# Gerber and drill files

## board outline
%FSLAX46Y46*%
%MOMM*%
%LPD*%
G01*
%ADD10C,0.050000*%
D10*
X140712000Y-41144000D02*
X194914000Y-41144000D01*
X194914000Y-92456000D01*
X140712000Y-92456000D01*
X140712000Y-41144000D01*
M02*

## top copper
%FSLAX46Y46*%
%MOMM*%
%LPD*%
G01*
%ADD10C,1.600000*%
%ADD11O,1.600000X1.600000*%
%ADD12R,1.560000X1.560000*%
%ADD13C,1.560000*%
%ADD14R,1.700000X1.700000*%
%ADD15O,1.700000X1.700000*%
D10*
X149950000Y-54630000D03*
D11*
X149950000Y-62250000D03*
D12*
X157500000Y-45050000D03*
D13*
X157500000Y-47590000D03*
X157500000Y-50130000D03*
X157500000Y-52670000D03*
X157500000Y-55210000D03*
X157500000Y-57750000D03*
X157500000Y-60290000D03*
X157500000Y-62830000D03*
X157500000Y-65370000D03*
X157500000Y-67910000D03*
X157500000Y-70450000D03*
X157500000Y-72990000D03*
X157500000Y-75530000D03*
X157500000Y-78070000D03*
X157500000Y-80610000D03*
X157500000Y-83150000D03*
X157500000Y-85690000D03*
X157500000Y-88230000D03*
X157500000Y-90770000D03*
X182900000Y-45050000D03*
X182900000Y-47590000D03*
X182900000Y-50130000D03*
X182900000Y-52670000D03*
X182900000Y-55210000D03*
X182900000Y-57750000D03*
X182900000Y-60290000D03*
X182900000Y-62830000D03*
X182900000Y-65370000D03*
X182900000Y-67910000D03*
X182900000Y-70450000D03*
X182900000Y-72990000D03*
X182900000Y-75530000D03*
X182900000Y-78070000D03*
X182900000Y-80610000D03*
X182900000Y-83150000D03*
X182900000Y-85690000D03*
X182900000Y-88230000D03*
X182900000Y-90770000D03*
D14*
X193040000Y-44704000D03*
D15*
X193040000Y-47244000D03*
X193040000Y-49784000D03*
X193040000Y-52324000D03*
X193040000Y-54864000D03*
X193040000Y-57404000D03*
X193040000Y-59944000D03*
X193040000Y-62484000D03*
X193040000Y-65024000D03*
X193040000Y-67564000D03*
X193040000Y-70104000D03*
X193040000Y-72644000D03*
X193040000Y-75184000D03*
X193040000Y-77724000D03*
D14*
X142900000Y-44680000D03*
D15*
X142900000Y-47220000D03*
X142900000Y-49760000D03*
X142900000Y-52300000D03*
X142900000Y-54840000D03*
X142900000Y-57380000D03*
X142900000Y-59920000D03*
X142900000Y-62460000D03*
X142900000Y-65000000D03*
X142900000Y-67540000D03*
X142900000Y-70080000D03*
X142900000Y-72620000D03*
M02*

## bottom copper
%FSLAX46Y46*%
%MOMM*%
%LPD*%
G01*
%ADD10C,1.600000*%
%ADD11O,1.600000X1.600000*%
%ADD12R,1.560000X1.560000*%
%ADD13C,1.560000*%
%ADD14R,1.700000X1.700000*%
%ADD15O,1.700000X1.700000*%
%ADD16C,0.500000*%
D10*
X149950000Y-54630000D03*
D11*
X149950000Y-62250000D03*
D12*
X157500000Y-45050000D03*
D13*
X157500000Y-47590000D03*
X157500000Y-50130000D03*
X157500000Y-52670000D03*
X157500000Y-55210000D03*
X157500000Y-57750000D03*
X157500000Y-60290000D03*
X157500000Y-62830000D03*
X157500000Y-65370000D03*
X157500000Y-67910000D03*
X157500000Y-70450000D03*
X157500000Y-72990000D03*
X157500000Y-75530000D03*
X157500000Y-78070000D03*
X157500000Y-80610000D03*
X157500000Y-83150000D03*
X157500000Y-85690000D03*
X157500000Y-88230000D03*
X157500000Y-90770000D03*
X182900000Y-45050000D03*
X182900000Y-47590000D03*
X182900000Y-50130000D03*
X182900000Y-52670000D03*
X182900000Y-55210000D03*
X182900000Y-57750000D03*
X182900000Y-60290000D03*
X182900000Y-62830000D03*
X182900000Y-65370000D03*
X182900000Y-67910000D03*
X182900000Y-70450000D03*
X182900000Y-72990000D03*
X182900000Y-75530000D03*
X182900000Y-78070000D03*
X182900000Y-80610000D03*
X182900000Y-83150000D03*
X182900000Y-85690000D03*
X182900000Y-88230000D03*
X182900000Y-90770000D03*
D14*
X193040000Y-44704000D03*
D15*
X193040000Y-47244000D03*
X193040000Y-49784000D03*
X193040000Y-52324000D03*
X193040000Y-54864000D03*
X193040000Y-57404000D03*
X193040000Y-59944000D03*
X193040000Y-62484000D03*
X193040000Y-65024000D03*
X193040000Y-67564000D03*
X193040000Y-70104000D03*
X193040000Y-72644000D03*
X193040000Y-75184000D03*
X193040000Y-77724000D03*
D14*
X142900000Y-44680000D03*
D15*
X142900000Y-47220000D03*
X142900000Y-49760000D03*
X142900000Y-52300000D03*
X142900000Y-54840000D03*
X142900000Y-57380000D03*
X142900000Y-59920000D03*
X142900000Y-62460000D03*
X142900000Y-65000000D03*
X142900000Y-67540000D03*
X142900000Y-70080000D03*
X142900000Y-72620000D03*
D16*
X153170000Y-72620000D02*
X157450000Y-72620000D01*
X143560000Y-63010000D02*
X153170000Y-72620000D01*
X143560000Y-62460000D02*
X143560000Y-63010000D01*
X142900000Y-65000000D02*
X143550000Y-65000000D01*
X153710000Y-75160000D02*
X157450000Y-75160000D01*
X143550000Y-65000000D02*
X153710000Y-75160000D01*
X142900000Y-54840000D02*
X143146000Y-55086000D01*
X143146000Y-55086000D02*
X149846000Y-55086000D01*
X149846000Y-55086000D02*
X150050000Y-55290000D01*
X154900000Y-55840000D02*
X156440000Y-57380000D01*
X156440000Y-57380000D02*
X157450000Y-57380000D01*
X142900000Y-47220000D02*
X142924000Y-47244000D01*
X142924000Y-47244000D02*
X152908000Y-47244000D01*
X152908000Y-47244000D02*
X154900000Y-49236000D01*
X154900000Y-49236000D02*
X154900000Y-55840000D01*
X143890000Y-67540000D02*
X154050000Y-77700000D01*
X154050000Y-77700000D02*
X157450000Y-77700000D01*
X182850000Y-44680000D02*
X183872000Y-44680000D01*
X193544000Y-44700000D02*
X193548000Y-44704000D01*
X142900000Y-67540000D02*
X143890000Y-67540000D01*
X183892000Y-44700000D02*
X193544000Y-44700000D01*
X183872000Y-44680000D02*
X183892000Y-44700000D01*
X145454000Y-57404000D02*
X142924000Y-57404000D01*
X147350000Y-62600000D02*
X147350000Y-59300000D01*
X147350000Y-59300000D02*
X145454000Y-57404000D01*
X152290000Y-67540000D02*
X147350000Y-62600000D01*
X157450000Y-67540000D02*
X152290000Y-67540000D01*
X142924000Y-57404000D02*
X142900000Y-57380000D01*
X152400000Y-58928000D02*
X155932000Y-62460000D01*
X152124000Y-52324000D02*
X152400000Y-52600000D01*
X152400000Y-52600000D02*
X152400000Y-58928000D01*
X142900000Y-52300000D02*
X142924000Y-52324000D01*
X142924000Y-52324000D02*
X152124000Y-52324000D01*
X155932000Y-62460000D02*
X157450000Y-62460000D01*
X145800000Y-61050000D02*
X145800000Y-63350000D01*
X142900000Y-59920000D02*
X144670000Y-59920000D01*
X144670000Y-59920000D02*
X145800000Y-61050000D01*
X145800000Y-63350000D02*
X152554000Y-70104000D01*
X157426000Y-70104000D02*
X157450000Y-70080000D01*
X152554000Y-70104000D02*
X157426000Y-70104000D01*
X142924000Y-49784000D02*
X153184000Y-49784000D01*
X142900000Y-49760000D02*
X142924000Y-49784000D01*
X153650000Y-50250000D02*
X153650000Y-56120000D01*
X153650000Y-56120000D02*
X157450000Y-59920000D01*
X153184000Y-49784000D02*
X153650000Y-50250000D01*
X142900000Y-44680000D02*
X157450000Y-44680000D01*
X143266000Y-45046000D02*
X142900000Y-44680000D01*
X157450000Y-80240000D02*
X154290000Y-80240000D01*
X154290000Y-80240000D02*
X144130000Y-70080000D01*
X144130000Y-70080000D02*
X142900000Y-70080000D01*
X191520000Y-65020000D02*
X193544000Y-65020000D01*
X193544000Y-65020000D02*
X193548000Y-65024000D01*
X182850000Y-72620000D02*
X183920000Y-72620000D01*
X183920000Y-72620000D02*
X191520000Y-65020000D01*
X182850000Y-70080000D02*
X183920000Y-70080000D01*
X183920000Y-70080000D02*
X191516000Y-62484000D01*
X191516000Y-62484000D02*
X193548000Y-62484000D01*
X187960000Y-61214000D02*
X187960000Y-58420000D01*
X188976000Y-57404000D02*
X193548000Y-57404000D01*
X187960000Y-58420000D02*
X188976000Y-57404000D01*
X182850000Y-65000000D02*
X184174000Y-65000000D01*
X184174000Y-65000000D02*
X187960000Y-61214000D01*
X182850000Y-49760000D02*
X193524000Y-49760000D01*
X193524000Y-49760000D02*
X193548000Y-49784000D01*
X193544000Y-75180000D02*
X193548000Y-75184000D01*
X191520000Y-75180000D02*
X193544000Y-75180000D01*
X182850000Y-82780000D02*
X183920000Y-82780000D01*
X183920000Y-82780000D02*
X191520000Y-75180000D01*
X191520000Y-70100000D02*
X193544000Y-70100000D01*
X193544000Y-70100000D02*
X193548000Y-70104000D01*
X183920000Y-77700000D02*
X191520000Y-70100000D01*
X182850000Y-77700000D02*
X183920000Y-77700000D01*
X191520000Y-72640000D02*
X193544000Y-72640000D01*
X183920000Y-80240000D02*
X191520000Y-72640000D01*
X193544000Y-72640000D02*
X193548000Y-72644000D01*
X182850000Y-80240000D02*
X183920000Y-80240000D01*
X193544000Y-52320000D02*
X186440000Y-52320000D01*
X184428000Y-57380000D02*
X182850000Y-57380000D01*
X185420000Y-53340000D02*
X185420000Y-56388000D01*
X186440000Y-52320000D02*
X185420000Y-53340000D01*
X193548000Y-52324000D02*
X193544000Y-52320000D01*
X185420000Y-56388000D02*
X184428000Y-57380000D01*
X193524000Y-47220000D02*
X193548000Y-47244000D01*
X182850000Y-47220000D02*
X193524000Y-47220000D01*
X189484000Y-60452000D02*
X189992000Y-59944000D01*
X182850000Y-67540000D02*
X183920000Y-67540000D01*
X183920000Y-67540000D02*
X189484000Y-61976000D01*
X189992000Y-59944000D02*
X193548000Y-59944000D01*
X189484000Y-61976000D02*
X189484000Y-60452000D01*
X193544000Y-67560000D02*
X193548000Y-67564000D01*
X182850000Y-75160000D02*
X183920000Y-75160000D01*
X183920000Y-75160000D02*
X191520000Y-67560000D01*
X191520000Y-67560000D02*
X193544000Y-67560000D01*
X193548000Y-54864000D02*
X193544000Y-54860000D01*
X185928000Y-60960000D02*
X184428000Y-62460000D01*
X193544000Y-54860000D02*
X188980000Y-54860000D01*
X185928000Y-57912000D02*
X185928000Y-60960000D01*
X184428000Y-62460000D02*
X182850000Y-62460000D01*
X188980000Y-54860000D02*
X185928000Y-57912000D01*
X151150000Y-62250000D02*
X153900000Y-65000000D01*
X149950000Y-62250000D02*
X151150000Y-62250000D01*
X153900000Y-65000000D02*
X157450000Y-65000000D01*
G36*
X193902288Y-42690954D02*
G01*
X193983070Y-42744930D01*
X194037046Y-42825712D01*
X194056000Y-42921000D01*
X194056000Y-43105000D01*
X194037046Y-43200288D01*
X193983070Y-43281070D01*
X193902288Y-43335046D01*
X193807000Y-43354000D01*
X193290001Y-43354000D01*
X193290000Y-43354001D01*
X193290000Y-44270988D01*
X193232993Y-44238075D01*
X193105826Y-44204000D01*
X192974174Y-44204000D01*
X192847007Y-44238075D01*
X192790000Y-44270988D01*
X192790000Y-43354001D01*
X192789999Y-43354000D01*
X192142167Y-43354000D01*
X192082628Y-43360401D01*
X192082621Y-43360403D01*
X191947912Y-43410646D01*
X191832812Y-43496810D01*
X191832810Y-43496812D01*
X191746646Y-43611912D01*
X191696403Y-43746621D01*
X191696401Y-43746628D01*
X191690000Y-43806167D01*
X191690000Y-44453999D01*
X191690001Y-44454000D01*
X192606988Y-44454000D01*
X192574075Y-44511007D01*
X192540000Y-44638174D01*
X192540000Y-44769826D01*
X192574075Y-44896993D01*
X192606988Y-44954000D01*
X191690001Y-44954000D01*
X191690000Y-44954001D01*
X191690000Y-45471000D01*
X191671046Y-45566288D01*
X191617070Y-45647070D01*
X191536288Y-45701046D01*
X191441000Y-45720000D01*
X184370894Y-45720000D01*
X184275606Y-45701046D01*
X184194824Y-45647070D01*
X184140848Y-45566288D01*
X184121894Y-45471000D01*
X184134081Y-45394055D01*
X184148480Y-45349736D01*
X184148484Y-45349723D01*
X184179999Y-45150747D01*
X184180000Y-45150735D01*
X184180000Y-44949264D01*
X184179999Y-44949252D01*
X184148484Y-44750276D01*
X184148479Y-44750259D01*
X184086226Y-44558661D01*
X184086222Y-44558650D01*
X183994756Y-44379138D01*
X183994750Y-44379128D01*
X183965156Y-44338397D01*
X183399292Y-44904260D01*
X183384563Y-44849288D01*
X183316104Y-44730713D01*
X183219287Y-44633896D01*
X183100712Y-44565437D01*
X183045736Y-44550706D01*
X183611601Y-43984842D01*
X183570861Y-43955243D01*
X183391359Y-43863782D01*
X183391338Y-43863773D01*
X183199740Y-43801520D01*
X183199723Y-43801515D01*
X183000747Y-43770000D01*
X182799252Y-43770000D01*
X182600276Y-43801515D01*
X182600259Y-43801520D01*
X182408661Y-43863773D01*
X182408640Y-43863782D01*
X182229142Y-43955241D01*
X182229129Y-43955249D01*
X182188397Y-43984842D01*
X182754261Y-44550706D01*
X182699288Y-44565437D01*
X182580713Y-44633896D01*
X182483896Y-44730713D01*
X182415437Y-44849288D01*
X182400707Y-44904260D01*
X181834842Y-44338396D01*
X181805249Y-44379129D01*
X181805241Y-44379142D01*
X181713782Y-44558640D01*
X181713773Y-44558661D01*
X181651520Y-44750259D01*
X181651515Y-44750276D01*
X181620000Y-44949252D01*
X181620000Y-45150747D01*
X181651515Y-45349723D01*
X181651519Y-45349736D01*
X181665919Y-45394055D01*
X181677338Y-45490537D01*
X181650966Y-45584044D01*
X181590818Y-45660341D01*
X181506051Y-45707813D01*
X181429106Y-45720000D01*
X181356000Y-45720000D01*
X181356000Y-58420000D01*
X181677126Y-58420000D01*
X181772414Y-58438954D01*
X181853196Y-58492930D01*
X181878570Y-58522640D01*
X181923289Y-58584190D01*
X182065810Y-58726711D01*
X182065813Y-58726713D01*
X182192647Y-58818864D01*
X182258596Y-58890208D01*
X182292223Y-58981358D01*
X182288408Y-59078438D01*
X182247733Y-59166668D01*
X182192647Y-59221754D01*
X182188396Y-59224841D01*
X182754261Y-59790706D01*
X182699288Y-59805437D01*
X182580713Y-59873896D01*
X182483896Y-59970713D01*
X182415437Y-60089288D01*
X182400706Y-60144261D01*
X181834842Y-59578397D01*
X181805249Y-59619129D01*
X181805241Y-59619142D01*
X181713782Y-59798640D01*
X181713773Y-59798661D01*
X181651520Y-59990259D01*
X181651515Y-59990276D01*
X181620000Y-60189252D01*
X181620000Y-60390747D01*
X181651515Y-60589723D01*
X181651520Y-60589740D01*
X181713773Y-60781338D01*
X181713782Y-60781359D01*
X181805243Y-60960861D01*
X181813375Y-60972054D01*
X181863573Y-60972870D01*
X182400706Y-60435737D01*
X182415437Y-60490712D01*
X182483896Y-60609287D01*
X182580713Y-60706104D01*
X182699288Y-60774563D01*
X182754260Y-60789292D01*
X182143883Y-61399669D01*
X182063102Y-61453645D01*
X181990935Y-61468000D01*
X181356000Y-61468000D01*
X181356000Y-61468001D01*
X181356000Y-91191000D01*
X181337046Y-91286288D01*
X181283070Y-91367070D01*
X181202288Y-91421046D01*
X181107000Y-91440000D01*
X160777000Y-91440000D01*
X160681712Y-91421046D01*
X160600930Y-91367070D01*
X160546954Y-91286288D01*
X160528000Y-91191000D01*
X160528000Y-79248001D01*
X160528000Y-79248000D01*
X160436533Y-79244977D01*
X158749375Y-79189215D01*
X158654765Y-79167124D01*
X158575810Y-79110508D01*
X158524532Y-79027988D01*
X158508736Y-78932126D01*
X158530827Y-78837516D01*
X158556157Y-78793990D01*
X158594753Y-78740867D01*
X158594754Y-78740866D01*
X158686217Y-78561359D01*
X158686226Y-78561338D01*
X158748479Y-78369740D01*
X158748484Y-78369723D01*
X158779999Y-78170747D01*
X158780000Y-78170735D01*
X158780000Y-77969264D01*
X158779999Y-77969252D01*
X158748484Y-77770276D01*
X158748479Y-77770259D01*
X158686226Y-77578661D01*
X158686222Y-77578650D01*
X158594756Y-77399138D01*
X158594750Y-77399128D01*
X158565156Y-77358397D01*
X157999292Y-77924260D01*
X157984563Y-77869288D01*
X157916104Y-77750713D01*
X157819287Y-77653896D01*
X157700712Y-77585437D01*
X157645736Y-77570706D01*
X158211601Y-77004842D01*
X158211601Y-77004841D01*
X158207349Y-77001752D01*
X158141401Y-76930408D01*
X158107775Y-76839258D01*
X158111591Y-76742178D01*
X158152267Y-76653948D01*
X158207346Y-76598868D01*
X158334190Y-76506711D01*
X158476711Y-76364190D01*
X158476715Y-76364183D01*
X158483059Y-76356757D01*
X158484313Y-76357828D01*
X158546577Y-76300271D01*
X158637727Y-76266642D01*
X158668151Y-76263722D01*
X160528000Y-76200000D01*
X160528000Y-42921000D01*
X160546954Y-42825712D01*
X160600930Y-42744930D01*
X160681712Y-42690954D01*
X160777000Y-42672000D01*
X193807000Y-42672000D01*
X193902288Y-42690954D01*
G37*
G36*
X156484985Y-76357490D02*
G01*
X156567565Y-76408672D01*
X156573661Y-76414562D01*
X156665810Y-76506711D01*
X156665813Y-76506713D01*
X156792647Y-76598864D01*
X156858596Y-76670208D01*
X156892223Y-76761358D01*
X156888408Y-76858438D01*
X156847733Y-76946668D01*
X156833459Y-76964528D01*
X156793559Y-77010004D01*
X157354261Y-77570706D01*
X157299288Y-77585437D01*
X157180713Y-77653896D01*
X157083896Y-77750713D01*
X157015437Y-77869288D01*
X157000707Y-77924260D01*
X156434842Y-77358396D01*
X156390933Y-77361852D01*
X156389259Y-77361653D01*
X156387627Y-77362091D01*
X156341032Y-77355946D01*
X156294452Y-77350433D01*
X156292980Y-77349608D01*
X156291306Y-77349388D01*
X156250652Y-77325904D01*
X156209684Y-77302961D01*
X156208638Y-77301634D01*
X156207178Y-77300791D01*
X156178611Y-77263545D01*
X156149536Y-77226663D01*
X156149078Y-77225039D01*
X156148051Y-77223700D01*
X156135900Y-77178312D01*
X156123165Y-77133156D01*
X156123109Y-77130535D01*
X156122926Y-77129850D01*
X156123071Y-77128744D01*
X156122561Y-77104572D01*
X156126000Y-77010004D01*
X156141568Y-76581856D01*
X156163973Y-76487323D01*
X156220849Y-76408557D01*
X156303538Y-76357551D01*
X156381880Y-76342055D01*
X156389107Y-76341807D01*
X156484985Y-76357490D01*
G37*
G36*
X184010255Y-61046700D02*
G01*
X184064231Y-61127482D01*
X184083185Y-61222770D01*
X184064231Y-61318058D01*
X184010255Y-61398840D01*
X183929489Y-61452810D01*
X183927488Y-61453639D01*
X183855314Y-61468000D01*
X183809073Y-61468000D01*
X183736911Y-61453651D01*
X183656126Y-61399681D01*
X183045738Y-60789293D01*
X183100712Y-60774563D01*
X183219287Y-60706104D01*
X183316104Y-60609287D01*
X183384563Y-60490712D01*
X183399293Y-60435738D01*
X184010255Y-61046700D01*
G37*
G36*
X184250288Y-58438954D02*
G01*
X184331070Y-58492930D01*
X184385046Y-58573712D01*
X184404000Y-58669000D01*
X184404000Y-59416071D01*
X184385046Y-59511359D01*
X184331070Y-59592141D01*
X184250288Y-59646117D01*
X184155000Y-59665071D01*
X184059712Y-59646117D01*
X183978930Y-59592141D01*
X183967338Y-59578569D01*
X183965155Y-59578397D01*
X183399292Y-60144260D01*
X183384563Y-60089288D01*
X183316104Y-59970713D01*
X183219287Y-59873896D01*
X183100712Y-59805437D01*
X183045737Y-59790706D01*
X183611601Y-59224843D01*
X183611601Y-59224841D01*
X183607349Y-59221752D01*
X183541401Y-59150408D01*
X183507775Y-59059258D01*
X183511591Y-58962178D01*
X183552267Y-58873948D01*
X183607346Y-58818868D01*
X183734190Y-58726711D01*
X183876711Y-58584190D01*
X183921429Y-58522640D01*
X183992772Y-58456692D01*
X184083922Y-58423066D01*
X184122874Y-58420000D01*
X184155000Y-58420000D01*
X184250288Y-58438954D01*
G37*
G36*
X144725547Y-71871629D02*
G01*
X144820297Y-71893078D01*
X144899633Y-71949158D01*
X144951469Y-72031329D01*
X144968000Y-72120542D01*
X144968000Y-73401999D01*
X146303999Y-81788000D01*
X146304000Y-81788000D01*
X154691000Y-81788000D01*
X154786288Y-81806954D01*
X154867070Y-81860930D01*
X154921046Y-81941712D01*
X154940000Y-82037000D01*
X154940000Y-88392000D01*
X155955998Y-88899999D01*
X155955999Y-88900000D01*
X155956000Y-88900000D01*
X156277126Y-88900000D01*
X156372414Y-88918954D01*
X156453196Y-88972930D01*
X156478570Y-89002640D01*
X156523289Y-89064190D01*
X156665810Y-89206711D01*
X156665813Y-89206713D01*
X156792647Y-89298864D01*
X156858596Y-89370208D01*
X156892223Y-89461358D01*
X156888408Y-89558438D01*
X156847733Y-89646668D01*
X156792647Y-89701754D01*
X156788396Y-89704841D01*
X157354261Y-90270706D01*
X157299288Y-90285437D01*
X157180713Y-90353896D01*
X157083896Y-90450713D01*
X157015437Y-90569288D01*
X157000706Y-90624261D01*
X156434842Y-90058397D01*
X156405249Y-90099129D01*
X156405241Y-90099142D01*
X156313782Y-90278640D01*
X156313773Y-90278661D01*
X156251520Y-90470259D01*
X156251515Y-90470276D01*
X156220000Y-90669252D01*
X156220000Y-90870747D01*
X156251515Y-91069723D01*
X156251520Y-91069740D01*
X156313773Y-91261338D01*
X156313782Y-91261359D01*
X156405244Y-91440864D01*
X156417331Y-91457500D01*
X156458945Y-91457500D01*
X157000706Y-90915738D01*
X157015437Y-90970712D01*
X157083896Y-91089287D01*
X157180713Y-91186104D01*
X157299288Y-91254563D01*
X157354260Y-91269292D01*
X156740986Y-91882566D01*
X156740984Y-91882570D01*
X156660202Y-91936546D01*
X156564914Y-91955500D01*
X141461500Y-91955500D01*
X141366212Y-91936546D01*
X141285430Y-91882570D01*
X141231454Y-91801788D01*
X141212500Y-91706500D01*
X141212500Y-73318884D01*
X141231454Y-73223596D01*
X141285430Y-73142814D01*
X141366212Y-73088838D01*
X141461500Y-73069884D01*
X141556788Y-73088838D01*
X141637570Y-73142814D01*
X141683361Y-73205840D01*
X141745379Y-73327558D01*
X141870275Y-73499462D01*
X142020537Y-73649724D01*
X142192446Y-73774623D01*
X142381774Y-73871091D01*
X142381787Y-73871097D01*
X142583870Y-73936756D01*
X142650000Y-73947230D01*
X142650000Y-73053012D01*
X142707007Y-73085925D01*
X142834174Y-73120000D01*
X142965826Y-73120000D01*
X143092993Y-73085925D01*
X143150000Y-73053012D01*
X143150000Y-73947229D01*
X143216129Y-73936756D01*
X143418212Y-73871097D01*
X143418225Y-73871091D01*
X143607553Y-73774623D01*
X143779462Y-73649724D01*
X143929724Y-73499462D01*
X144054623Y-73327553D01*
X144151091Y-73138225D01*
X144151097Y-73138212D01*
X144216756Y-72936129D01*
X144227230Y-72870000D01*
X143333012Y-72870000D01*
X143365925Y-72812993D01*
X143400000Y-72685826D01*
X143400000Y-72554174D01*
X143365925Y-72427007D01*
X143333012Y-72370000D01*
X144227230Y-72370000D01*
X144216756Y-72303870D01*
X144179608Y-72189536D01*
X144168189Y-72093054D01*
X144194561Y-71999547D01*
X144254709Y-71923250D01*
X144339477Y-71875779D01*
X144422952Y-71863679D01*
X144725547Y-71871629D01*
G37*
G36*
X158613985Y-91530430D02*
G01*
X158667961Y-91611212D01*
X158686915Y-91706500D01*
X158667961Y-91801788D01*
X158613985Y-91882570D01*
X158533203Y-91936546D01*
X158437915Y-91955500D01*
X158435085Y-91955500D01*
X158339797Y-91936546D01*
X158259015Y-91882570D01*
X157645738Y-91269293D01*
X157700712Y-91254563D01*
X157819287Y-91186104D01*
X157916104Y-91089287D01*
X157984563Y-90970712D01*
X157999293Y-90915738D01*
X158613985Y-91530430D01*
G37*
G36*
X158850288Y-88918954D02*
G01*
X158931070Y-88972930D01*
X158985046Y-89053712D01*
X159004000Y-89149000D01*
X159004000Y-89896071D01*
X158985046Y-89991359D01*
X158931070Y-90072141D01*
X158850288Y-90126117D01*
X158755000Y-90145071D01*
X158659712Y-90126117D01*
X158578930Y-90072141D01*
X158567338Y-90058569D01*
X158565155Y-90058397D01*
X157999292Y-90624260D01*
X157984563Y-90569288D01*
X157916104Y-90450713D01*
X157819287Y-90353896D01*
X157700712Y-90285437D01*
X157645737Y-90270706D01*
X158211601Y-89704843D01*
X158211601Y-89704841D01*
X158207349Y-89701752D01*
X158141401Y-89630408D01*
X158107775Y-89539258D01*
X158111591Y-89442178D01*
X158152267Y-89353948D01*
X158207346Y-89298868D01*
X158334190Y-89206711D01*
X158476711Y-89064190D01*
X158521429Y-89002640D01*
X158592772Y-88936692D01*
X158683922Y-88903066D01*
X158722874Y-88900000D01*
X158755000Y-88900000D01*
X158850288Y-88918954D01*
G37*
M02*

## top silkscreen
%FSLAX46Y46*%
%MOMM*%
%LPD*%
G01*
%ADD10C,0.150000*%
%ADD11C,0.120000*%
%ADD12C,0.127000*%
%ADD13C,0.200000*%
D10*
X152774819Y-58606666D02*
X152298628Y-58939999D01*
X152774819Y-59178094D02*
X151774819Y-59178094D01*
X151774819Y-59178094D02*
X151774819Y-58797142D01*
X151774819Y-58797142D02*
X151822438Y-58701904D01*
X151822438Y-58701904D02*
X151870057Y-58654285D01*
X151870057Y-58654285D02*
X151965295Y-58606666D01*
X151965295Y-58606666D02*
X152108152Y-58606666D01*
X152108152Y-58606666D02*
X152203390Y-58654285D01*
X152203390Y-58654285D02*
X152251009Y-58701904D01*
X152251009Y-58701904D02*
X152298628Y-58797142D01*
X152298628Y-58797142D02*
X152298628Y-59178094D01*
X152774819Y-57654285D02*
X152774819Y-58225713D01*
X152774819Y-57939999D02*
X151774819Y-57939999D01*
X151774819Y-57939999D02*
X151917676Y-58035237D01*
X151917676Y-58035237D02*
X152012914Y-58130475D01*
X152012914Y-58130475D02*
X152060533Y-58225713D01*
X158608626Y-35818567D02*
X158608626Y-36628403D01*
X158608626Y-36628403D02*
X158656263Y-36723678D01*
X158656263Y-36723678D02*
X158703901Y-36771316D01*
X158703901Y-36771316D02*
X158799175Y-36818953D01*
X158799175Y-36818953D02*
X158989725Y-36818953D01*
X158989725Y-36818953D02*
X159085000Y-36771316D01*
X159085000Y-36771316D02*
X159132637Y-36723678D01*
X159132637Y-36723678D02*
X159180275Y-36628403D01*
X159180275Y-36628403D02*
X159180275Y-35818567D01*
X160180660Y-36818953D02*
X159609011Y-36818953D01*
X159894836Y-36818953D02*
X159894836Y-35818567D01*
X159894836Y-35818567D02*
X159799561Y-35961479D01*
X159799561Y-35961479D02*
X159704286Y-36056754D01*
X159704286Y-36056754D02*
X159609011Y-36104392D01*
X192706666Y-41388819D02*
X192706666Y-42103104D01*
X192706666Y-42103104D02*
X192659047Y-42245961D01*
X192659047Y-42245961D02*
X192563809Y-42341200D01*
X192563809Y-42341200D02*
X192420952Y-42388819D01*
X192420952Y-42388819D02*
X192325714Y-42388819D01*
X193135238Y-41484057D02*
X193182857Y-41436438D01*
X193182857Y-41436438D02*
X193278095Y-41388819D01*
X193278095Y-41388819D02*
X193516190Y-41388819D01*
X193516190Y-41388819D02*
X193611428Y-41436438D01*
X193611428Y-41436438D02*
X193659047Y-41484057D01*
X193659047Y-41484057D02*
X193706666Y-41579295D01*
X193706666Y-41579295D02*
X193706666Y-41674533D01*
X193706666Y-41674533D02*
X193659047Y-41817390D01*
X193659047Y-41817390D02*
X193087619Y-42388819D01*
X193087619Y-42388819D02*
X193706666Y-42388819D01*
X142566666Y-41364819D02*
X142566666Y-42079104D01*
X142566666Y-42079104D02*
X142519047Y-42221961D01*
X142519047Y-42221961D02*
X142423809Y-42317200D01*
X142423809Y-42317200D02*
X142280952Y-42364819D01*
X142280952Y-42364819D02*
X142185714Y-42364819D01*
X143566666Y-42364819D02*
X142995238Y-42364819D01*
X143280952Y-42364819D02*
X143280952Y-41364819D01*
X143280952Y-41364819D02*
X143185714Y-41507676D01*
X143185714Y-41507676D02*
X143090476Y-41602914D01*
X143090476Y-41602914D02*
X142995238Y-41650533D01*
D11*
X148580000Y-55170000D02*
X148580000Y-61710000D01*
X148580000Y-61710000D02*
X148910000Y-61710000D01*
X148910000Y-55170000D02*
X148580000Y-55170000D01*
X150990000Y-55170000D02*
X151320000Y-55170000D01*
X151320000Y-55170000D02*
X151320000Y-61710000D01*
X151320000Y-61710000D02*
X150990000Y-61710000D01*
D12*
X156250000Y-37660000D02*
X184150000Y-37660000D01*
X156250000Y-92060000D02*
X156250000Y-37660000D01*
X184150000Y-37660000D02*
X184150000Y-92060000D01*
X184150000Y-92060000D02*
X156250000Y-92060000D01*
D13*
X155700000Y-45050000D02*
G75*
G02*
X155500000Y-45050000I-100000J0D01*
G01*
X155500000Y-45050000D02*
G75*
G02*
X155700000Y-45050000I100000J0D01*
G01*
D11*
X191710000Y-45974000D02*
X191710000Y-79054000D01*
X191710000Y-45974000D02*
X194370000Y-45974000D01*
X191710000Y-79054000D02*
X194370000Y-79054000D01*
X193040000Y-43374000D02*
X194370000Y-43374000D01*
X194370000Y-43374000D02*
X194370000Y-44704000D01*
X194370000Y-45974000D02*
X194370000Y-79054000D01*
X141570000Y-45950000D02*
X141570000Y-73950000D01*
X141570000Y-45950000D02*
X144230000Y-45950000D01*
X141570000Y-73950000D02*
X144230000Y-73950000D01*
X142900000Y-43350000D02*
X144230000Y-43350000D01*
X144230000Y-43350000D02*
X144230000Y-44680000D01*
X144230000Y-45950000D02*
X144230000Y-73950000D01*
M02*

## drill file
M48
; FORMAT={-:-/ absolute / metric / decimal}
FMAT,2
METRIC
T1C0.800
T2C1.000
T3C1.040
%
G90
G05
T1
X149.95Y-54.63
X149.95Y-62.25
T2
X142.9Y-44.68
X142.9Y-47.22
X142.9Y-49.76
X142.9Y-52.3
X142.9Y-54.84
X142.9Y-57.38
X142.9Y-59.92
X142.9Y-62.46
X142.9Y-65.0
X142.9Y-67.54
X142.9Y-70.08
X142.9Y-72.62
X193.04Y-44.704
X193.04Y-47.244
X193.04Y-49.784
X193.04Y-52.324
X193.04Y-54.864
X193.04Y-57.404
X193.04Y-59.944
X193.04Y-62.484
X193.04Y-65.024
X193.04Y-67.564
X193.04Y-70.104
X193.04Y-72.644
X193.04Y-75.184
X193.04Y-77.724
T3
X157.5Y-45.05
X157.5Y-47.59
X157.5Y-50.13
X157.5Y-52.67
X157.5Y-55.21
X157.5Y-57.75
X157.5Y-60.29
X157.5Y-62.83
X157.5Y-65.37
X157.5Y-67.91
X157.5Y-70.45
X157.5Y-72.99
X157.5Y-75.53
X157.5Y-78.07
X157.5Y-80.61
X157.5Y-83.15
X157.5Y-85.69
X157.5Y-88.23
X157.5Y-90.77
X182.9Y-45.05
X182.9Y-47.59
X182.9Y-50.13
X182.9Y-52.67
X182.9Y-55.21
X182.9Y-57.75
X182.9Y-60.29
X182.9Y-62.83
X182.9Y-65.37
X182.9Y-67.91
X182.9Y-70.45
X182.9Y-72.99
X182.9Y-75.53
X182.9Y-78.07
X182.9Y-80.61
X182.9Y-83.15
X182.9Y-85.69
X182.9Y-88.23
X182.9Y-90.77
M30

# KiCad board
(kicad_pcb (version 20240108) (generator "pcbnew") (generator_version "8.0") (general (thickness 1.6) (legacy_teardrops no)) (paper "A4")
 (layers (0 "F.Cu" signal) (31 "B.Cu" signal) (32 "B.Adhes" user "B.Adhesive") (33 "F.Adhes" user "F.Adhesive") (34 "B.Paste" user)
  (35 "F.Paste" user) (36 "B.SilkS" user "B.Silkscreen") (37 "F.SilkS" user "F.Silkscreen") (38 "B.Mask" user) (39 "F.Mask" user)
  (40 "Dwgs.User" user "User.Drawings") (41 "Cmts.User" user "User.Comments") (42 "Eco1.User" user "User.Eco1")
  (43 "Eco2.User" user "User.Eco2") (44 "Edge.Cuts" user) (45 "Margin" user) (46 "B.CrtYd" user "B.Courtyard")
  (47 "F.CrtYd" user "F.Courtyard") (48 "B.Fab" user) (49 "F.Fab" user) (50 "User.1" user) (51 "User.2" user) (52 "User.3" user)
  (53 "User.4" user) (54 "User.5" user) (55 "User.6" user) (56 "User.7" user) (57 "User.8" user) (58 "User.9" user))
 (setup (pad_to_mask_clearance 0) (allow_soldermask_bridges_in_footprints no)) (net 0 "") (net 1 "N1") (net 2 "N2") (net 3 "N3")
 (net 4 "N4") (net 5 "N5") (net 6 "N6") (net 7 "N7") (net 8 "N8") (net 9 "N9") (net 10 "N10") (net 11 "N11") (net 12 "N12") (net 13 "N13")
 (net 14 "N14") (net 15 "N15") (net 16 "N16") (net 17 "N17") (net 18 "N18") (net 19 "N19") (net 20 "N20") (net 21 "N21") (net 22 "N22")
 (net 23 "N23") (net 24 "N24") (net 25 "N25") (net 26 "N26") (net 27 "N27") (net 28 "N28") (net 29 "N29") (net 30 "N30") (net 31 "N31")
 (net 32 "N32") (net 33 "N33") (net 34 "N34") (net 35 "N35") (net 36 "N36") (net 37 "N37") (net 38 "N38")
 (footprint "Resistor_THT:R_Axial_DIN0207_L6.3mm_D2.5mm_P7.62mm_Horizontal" (layer "F.Cu") (at 149.95 54.63 -90)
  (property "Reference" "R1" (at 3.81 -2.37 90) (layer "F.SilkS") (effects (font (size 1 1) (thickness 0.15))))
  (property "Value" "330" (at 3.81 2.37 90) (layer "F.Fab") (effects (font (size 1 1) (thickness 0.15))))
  (fp_line (start 0.54 1.37) (end 7.08 1.37) (stroke (width 0.12) (type solid)) (layer "F.SilkS"))
  (fp_line (start 7.08 1.37) (end 7.08 1.04) (stroke (width 0.12) (type solid)) (layer "F.SilkS"))
  (fp_line (start 0.54 1.04) (end 0.54 1.37) (stroke (width 0.12) (type solid)) (layer "F.SilkS"))
  (fp_line (start 0.54 -1.04) (end 0.54 -1.37) (stroke (width 0.12) (type solid)) (layer "F.SilkS"))
  (fp_line (start 0.54 -1.37) (end 7.08 -1.37) (stroke (width 0.12) (type solid)) (layer "F.SilkS"))
  (fp_line (start 7.08 -1.37) (end 7.08 -1.04) (stroke (width 0.12) (type solid)) (layer "F.SilkS"))
  (pad "1" thru_hole circle (at 0 0 270) (size 1.6 1.6) (drill 0.8) (layers "*.Cu" "*.Mask") (remove_unused_layers no) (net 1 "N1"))
  (pad "2" thru_hole oval (at 7.62 0 270) (size 1.6 1.6) (drill 0.8) (layers "*.Cu" "*.Mask") (remove_unused_layers no) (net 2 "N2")))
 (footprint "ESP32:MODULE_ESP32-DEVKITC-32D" (layer "F.Cu") (at 170.2 64.81)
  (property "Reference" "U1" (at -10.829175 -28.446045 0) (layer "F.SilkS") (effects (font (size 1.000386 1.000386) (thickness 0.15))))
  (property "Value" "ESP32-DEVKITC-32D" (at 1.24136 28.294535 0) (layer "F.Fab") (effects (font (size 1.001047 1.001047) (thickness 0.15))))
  (fp_line (start -13.95 -27.15) (end 13.95 -27.15) (stroke (width 0.127) (type solid)) (layer "F.SilkS"))
  (fp_line (start -13.95 27.25) (end -13.95 -27.15) (stroke (width 0.127) (type solid)) (layer "F.SilkS"))
  (fp_line (start 13.95 -27.15) (end 13.95 27.25) (stroke (width 0.127) (type solid)) (layer "F.SilkS"))
  (fp_line (start 13.95 27.25) (end -13.95 27.25) (stroke (width 0.127) (type solid)) (layer "F.SilkS"))
  (fp_circle (center -14.6 -19.76) (end -14.5 -19.76) (stroke (width 0.2) (type solid)) (fill none) (layer "F.SilkS"))
  (pad "J2-1" thru_hole rect (at -12.7 -19.76) (size 1.56 1.56) (drill 1.04) (layers "*.Cu" "*.Mask") (remove_unused_layers no) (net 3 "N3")
   (solder_mask_margin 0.102))
  (pad "J2-2" thru_hole circle (at -12.7 -17.22) (size 1.56 1.56) (drill 1.04) (layers "*.Cu" "*.Mask") (remove_unused_layers no)
   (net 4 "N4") (solder_mask_margin 0.102))
  (pad "J2-3" thru_hole circle (at -12.7 -14.68) (size 1.56 1.56) (drill 1.04) (layers "*.Cu" "*.Mask") (remove_unused_layers no)
   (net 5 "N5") (solder_mask_margin 0.102))
  (pad "J2-4" thru_hole circle (at -12.7 -12.14) (size 1.56 1.56) (drill 1.04) (layers "*.Cu" "*.Mask") (remove_unused_layers no)
   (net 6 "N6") (solder_mask_margin 0.102))
  (pad "J2-5" thru_hole circle (at -12.7 -9.6) (size 1.56 1.56) (drill 1.04) (layers "*.Cu" "*.Mask") (remove_unused_layers no) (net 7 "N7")
   (solder_mask_margin 0.102))
  (pad "J2-6" thru_hole circle (at -12.7 -7.06) (size 1.56 1.56) (drill 1.04) (layers "*.Cu" "*.Mask") (remove_unused_layers no)
   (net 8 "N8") (solder_mask_margin 0.102))
  (pad "J2-7" thru_hole circle (at -12.7 -4.52) (size 1.56 1.56) (drill 1.04) (layers "*.Cu" "*.Mask") (remove_unused_layers no)
   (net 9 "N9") (solder_mask_margin 0.102))
  (pad "J2-8" thru_hole circle (at -12.7 -1.98) (size 1.56 1.56) (drill 1.04) (layers "*.Cu" "*.Mask") (remove_unused_layers no)
   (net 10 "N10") (solder_mask_margin 0.102))
  (pad "J2-9" thru_hole circle (at -12.7 0.56) (size 1.56 1.56) (drill 1.04) (layers "*.Cu" "*.Mask") (remove_unused_layers no) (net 2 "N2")
   (solder_mask_margin 0.102))
  (pad "J2-10" thru_hole circle (at -12.7 3.1) (size 1.56 1.56) (drill 1.04) (layers "*.Cu" "*.Mask") (remove_unused_layers no)
   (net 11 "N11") (solder_mask_margin 0.102))
  (pad "J2-11" thru_hole circle (at -12.7 5.64) (size 1.56 1.56) (drill 1.04) (layers "*.Cu" "*.Mask") (remove_unused_layers no)
   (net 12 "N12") (solder_mask_margin 0.102))
  (pad "J2-12" thru_hole circle (at -12.7 8.18) (size 1.56 1.56) (drill 1.04) (layers "*.Cu" "*.Mask") (remove_unused_layers no)
   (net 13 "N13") (solder_mask_margin 0.102))
  (pad "J2-13" thru_hole circle (at -12.7 10.72) (size 1.56 1.56) (drill 1.04) (layers "*.Cu" "*.Mask") (remove_unused_layers no)
   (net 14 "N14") (solder_mask_margin 0.102))
  (pad "J2-14" thru_hole circle (at -12.7 13.26) (size 1.56 1.56) (drill 1.04) (layers "*.Cu" "*.Mask") (remove_unused_layers no)
   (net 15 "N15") (solder_mask_margin 0.102))
  (pad "J2-15" thru_hole circle (at -12.7 15.8) (size 1.56 1.56) (drill 1.04) (layers "*.Cu" "*.Mask") (remove_unused_layers no)
   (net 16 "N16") (solder_mask_margin 0.102))
  (pad "J2-16" thru_hole circle (at -12.7 18.34) (size 1.56 1.56) (drill 1.04) (layers "*.Cu" "*.Mask") (remove_unused_layers no)
   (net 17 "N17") (solder_mask_margin 0.102))
  (pad "J2-17" thru_hole circle (at -12.7 20.88) (size 1.56 1.56) (drill 1.04) (layers "*.Cu" "*.Mask") (remove_unused_layers no)
   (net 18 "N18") (solder_mask_margin 0.102))
  (pad "J2-18" thru_hole circle (at -12.7 23.42) (size 1.56 1.56) (drill 1.04) (layers "*.Cu" "*.Mask") (remove_unused_layers no)
   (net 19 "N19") (solder_mask_margin 0.102))
  (pad "J2-19" thru_hole circle (at -12.7 25.96) (size 1.56 1.56) (drill 1.04) (layers "*.Cu" "*.Mask") (remove_unused_layers no)
   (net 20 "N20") (solder_mask_margin 0.102))
  (pad "J3-1" thru_hole circle (at 12.7 -19.76) (size 1.56 1.56) (drill 1.04) (layers "*.Cu" "*.Mask") (remove_unused_layers no)
   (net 15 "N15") (solder_mask_margin 0.102))
  (pad "J3-2" thru_hole circle (at 12.7 -17.22) (size 1.56 1.56) (drill 1.04) (layers "*.Cu" "*.Mask") (remove_unused_layers no)
   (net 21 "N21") (solder_mask_margin 0.102))
  (pad "J3-3" thru_hole circle (at 12.7 -14.68) (size 1.56 1.56) (drill 1.04) (layers "*.Cu" "*.Mask") (remove_unused_layers no)
   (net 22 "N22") (solder_mask_margin 0.102))
  (pad "J3-4" thru_hole circle (at 12.7 -12.14) (size 1.56 1.56) (drill 1.04) (layers "*.Cu" "*.Mask") (remove_unused_layers no)
   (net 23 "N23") (solder_mask_margin 0.102))
  (pad "J3-5" thru_hole circle (at 12.7 -9.6) (size 1.56 1.56) (drill 1.04) (layers "*.Cu" "*.Mask") (remove_unused_layers no)
   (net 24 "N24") (solder_mask_margin 0.102))
  (pad "J3-6" thru_hole circle (at 12.7 -7.06) (size 1.56 1.56) (drill 1.04) (layers "*.Cu" "*.Mask") (remove_unused_layers no)
   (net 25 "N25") (solder_mask_margin 0.102))
  (pad "J3-7" thru_hole circle (at 12.7 -4.52) (size 1.56 1.56) (drill 1.04) (layers "*.Cu" "*.Mask") (remove_unused_layers no)
   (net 15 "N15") (solder_mask_margin 0.102))
  (pad "J3-8" thru_hole circle (at 12.7 -1.98) (size 1.56 1.56) (drill 1.04) (layers "*.Cu" "*.Mask") (remove_unused_layers no)
   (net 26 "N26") (solder_mask_margin 0.102))
  (pad "J3-9" thru_hole circle (at 12.7 0.56) (size 1.56 1.56) (drill 1.04) (layers "*.Cu" "*.Mask") (remove_unused_layers no)
   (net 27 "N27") (solder_mask_margin 0.102))
  (pad "J3-10" thru_hole circle (at 12.7 3.1) (size 1.56 1.56) (drill 1.04) (layers "*.Cu" "*.Mask") (remove_unused_layers no)
   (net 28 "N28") (solder_mask_margin 0.102))
  (pad "J3-11" thru_hole circle (at 12.7 5.64) (size 1.56 1.56) (drill 1.04) (layers "*.Cu" "*.Mask") (remove_unused_layers no)
   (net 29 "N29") (solder_mask_margin 0.102))
  (pad "J3-12" thru_hole circle (at 12.7 8.18) (size 1.56 1.56) (drill 1.04) (layers "*.Cu" "*.Mask") (remove_unused_layers no)
   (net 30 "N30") (solder_mask_margin 0.102))
  (pad "J3-13" thru_hole circle (at 12.7 10.72) (size 1.56 1.56) (drill 1.04) (layers "*.Cu" "*.Mask") (remove_unused_layers no)
   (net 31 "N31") (solder_mask_margin 0.102))
  (pad "J3-14" thru_hole circle (at 12.7 13.26) (size 1.56 1.56) (drill 1.04) (layers "*.Cu" "*.Mask") (remove_unused_layers no)
   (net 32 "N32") (solder_mask_margin 0.102))
  (pad "J3-15" thru_hole circle (at 12.7 15.8) (size 1.56 1.56) (drill 1.04) (layers "*.Cu" "*.Mask") (remove_unused_layers no)
   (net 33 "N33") (solder_mask_margin 0.102))
  (pad "J3-16" thru_hole circle (at 12.7 18.34) (size 1.56 1.56) (drill 1.04) (layers "*.Cu" "*.Mask") (remove_unused_layers no)
   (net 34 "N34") (solder_mask_margin 0.102))
  (pad "J3-17" thru_hole circle (at 12.7 20.88) (size 1.56 1.56) (drill 1.04) (layers "*.Cu" "*.Mask") (remove_unused_layers no)
   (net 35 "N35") (solder_mask_margin 0.102))
  (pad "J3-18" thru_hole circle (at 12.7 23.42) (size 1.56 1.56) (drill 1.04) (layers "*.Cu" "*.Mask") (remove_unused_layers no)
   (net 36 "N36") (solder_mask_margin 0.102))
  (pad "J3-19" thru_hole circle (at 12.7 25.96) (size 1.56 1.56) (drill 1.04) (layers "*.Cu" "*.Mask") (remove_unused_layers no)
   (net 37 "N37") (solder_mask_margin 0.102)))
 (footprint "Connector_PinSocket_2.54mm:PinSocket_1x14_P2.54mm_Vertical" (layer "F.Cu") (at 193.04 44.704)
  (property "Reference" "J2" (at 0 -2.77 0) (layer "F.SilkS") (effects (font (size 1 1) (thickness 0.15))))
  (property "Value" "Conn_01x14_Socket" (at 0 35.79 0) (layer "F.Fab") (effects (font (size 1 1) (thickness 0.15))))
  (fp_line (start -1.33 1.27) (end -1.33 34.35) (stroke (width 0.12) (type solid)) (layer "F.SilkS"))
  (fp_line (start -1.33 1.27) (end 1.33 1.27) (stroke (width 0.12) (type solid)) (layer "F.SilkS"))
  (fp_line (start -1.33 34.35) (end 1.33 34.35) (stroke (width 0.12) (type solid)) (layer "F.SilkS"))
  (fp_line (start 0 -1.33) (end 1.33 -1.33) (stroke (width 0.12) (type solid)) (layer "F.SilkS"))
  (fp_line (start 1.33 -1.33) (end 1.33 0) (stroke (width 0.12) (type solid)) (layer "F.SilkS"))
  (fp_line (start 1.33 1.27) (end 1.33 34.35) (stroke (width 0.12) (type solid)) (layer "F.SilkS"))
  (pad "1" thru_hole rect (at 0 0) (size 1.7 1.7) (drill 1) (layers "*.Cu" "*.Mask") (remove_unused_layers no) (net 15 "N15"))
  (pad "2" thru_hole oval (at 0 2.54) (size 1.7 1.7) (drill 1) (layers "*.Cu" "*.Mask") (remove_unused_layers no) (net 21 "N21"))
  (pad "3" thru_hole oval (at 0 5.08) (size 1.7 1.7) (drill 1) (layers "*.Cu" "*.Mask") (remove_unused_layers no) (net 22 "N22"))
  (pad "4" thru_hole oval (at 0 7.62) (size 1.7 1.7) (drill 1) (layers "*.Cu" "*.Mask") (remove_unused_layers no) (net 25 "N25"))
  (pad "5" thru_hole oval (at 0 10.16) (size 1.7 1.7) (drill 1) (layers "*.Cu" "*.Mask") (remove_unused_layers no) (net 26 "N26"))
  (pad "6" thru_hole oval (at 0 12.7) (size 1.7 1.7) (drill 1) (layers "*.Cu" "*.Mask") (remove_unused_layers no) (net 27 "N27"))
  (pad "7" thru_hole oval (at 0 15.24) (size 1.7 1.7) (drill 1) (layers "*.Cu" "*.Mask") (remove_unused_layers no) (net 28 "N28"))
  (pad "8" thru_hole oval (at 0 17.78) (size 1.7 1.7) (drill 1) (layers "*.Cu" "*.Mask") (remove_unused_layers no) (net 29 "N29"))
  (pad "9" thru_hole oval (at 0 20.32) (size 1.7 1.7) (drill 1) (layers "*.Cu" "*.Mask") (remove_unused_layers no) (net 30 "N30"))
  (pad "10" thru_hole oval (at 0 22.86) (size 1.7 1.7) (drill 1) (layers "*.Cu" "*.Mask") (remove_unused_layers no) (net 31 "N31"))
  (pad "11" thru_hole oval (at 0 25.4) (size 1.7 1.7) (drill 1) (layers "*.Cu" "*.Mask") (remove_unused_layers no) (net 32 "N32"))
  (pad "12" thru_hole oval (at 0 27.94) (size 1.7 1.7) (drill 1) (layers "*.Cu" "*.Mask") (remove_unused_layers no) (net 33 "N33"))
  (pad "13" thru_hole oval (at 0 30.48) (size 1.7 1.7) (drill 1) (layers "*.Cu" "*.Mask") (remove_unused_layers no) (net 34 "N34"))
  (pad "14" thru_hole oval (at 0 33.02) (size 1.7 1.7) (drill 1) (layers "*.Cu" "*.Mask") (remove_unused_layers no) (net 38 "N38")))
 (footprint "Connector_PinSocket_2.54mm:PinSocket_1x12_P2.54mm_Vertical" (layer "F.Cu") (at 142.9 44.68)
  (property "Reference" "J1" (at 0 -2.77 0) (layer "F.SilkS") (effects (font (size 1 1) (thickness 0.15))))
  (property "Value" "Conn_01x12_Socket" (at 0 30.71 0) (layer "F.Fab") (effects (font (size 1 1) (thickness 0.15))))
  (fp_line (start -1.33 1.27) (end -1.33 29.27) (stroke (width 0.12) (type solid)) (layer "F.SilkS"))
  (fp_line (start -1.33 1.27) (end 1.33 1.27) (stroke (width 0.12) (type solid)) (layer "F.SilkS"))
  (fp_line (start -1.33 29.27) (end 1.33 29.27) (stroke (width 0.12) (type solid)) (layer "F.SilkS"))
  (fp_line (start 0 -1.33) (end 1.33 -1.33) (stroke (width 0.12) (type solid)) (layer "F.SilkS"))
  (fp_line (start 1.33 -1.33) (end 1.33 0) (stroke (width 0.12) (type solid)) (layer "F.SilkS"))
  (fp_line (start 1.33 1.27) (end 1.33 29.27) (stroke (width 0.12) (type solid)) (layer "F.SilkS"))
  (pad "1" thru_hole rect (at 0 0) (size 1.7 1.7) (drill 1) (layers "*.Cu" "*.Mask") (remove_unused_layers no) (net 3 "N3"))
  (pad "2" thru_hole oval (at 0 2.54) (size 1.7 1.7) (drill 1) (layers "*.Cu" "*.Mask") (remove_unused_layers no) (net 8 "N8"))
  (pad "3" thru_hole oval (at 0 5.08) (size 1.7 1.7) (drill 1) (layers "*.Cu" "*.Mask") (remove_unused_layers no) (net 9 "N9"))
  (pad "4" thru_hole oval (at 0 7.62) (size 1.7 1.7) (drill 1) (layers "*.Cu" "*.Mask") (remove_unused_layers no) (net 10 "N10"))
  (pad "5" thru_hole oval (at 0 10.16) (size 1.7 1.7) (drill 1) (layers "*.Cu" "*.Mask") (remove_unused_layers no) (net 1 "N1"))
  (pad "6" thru_hole oval (at 0 12.7) (size 1.7 1.7) (drill 1) (layers "*.Cu" "*.Mask") (remove_unused_layers no) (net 11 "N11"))
  (pad "7" thru_hole oval (at 0 15.24) (size 1.7 1.7) (drill 1) (layers "*.Cu" "*.Mask") (remove_unused_layers no) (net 12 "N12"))
  (pad "8" thru_hole oval (at 0 17.78) (size 1.7 1.7) (drill 1) (layers "*.Cu" "*.Mask") (remove_unused_layers no) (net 13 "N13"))
  (pad "9" thru_hole oval (at 0 20.32) (size 1.7 1.7) (drill 1) (layers "*.Cu" "*.Mask") (remove_unused_layers no) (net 14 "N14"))
  (pad "10" thru_hole oval (at 0 22.86) (size 1.7 1.7) (drill 1) (layers "*.Cu" "*.Mask") (remove_unused_layers no) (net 15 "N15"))
  (pad "11" thru_hole oval (at 0 25.4) (size 1.7 1.7) (drill 1) (layers "*.Cu" "*.Mask") (remove_unused_layers no) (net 16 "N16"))
  (pad "12" thru_hole oval (at 0 27.94) (size 1.7 1.7) (drill 1) (layers "*.Cu" "*.Mask") (remove_unused_layers no) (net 20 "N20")))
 (gr_rect (start 140.712 41.144) (end 194.914 92.456) (stroke (width 0.05) (type default)) (fill none) (layer "Edge.Cuts"))
 (segment (start 153.17 72.62) (end 157.45 72.62) (width 0.5) (layer "B.Cu") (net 13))
 (segment (start 143.56 63.01) (end 153.17 72.62) (width 0.5) (layer "B.Cu") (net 13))
 (segment (start 143.56 62.46) (end 143.56 63.01) (width 0.5) (layer "B.Cu") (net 13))
 (segment (start 142.9 65) (end 143.55 65) (width 0.5) (layer "B.Cu") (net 14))
 (segment (start 153.71 75.16) (end 157.45 75.16) (width 0.5) (layer "B.Cu") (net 14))
 (segment (start 143.55 65) (end 153.71 75.16) (width 0.5) (layer "B.Cu") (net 14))
 (segment (start 142.9 54.84) (end 143.146 55.086) (width 0.5) (layer "B.Cu") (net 1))
 (segment (start 143.146 55.086) (end 149.846 55.086) (width 0.5) (layer "B.Cu") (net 1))
 (segment (start 149.846 55.086) (end 150.05 55.29) (width 0.5) (layer "B.Cu") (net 1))
 (segment (start 154.9 55.84) (end 156.44 57.38) (width 0.5) (layer "B.Cu") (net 8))
 (segment (start 156.44 57.38) (end 157.45 57.38) (width 0.5) (layer "B.Cu") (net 8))
 (segment (start 142.9 47.22) (end 142.924 47.244) (width 0.5) (layer "B.Cu") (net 8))
 (segment (start 142.924 47.244) (end 152.908 47.244) (width 0.5) (layer "B.Cu") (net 8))
 (segment (start 152.908 47.244) (end 154.9 49.236) (width 0.5) (layer "B.Cu") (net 8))
 (segment (start 154.9 49.236) (end 154.9 55.84) (width 0.5) (layer "B.Cu") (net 8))
 (segment (start 143.89 67.54) (end 154.05 77.7) (width 0.5) (layer "B.Cu") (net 15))
 (segment (start 154.05 77.7) (end 157.45 77.7) (width 0.5) (layer "B.Cu") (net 15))
 (segment (start 182.85 44.68) (end 183.872 44.68) (width 0.5) (layer "B.Cu") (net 15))
 (segment (start 193.544 44.7) (end 193.548 44.704) (width 0.5) (layer "B.Cu") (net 15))
 (segment (start 142.9 67.54) (end 143.89 67.54) (width 0.5) (layer "B.Cu") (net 15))
 (segment (start 183.892 44.7) (end 193.544 44.7) (width 0.5) (layer "B.Cu") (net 15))
 (segment (start 183.872 44.68) (end 183.892 44.7) (width 0.5) (layer "B.Cu") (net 15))
 (segment (start 145.454 57.404) (end 142.924 57.404) (width 0.5) (layer "B.Cu") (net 11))
 (segment (start 147.35 62.6) (end 147.35 59.3) (width 0.5) (layer "B.Cu") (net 11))
 (segment (start 147.35 59.3) (end 145.454 57.404) (width 0.5) (layer "B.Cu") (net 11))
 (segment (start 152.29 67.54) (end 147.35 62.6) (width 0.5) (layer "B.Cu") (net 11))
 (segment (start 157.45 67.54) (end 152.29 67.54) (width 0.5) (layer "B.Cu") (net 11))
 (segment (start 142.924 57.404) (end 142.9 57.38) (width 0.5) (layer "B.Cu") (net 11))
 (segment (start 152.4 58.928) (end 155.932 62.46) (width 0.5) (layer "B.Cu") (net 10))
 (segment (start 152.124 52.324) (end 152.4 52.6) (width 0.5) (layer "B.Cu") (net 10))
 (segment (start 152.4 52.6) (end 152.4 58.928) (width 0.5) (layer "B.Cu") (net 10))
 (segment (start 142.9 52.3) (end 142.924 52.324) (width 0.5) (layer "B.Cu") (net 10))
 (segment (start 142.924 52.324) (end 152.124 52.324) (width 0.5) (layer "B.Cu") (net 10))
 (segment (start 155.932 62.46) (end 157.45 62.46) (width 0.5) (layer "B.Cu") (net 10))
 (segment (start 145.8 61.05) (end 145.8 63.35) (width 0.5) (layer "B.Cu") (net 12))
 (segment (start 142.9 59.92) (end 144.67 59.92) (width 0.5) (layer "B.Cu") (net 12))
 (segment (start 144.67 59.92) (end 145.8 61.05) (width 0.5) (layer "B.Cu") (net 12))
 (segment (start 145.8 63.35) (end 152.554 70.104) (width 0.5) (layer "B.Cu") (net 12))
 (segment (start 157.426 70.104) (end 157.45 70.08) (width 0.5) (layer "B.Cu") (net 12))
 (segment (start 152.554 70.104) (end 157.426 70.104) (width 0.5) (layer "B.Cu") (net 12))
 (segment (start 142.924 49.784) (end 153.184 49.784) (width 0.5) (layer "B.Cu") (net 9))
 (segment (start 142.9 49.76) (end 142.924 49.784) (width 0.5) (layer "B.Cu") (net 9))
 (segment (start 153.65 50.25) (end 153.65 56.12) (width 0.5) (layer "B.Cu") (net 9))
 (segment (start 153.65 56.12) (end 157.45 59.92) (width 0.5) (layer "B.Cu") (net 9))
 (segment (start 153.184 49.784) (end 153.65 50.25) (width 0.5) (layer "B.Cu") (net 9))
 (segment (start 142.9 44.68) (end 157.45 44.68) (width 0.5) (layer "B.Cu") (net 3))
 (segment (start 143.266 45.046) (end 142.9 44.68) (width 0.5) (layer "B.Cu") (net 3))
 (segment (start 157.45 80.24) (end 154.29 80.24) (width 0.5) (layer "B.Cu") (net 16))
 (segment (start 154.29 80.24) (end 144.13 70.08) (width 0.5) (layer "B.Cu") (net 16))
 (segment (start 144.13 70.08) (end 142.9 70.08) (width 0.5) (layer "B.Cu") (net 16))
 (segment (start 191.52 65.02) (end 193.544 65.02) (width 0.5) (layer "B.Cu") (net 30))
 (segment (start 193.544 65.02) (end 193.548 65.024) (width 0.5) (layer "B.Cu") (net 30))
 (segment (start 182.85 72.62) (end 183.92 72.62) (width 0.5) (layer "B.Cu") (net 30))
 (segment (start 183.92 72.62) (end 191.52 65.02) (width 0.5) (layer "B.Cu") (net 30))
 (segment (start 182.85 70.08) (end 183.92 70.08) (width 0.5) (layer "B.Cu") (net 29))
 (segment (start 183.92 70.08) (end 191.516 62.484) (width 0.5) (layer "B.Cu") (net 29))
 (segment (start 191.516 62.484) (end 193.548 62.484) (width 0.5) (layer "B.Cu") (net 29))
 (segment (start 187.96 61.214) (end 187.96 58.42) (width 0.5) (layer "B.Cu") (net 27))
 (segment (start 188.976 57.404) (end 193.548 57.404) (width 0.5) (layer "B.Cu") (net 27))
 (segment (start 187.96 58.42) (end 188.976 57.404) (width 0.5) (layer "B.Cu") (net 27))
 (segment (start 182.85 65) (end 184.174 65) (width 0.5) (layer "B.Cu") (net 27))
 (segment (start 184.174 65) (end 187.96 61.214) (width 0.5) (layer "B.Cu") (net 27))
 (segment (start 182.85 49.76) (end 193.524 49.76) (width 0.5) (layer "B.Cu") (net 22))
 (segment (start 193.524 49.76) (end 193.548 49.784) (width 0.5) (layer "B.Cu") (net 22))
 (segment (start 193.544 75.18) (end 193.548 75.184) (width 0.5) (layer "B.Cu") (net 34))
 (segment (start 191.52 75.18) (end 193.544 75.18) (width 0.5) (layer "B.Cu") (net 34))
 (segment (start 182.85 82.78) (end 183.92 82.78) (width 0.5) (layer "B.Cu") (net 34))
 (segment (start 183.92 82.78) (end 191.52 75.18) (width 0.5) (layer "B.Cu") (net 34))
 (segment (start 191.52 70.1) (end 193.544 70.1) (width 0.5) (layer "B.Cu") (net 32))
 (segment (start 193.544 70.1) (end 193.548 70.104) (width 0.5) (layer "B.Cu") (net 32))
 (segment (start 183.92 77.7) (end 191.52 70.1) (width 0.5) (layer "B.Cu") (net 32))
 (segment (start 182.85 77.7) (end 183.92 77.7) (width 0.5) (layer "B.Cu") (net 32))
 (segment (start 191.52 72.64) (end 193.544 72.64) (width 0.5) (layer "B.Cu") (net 33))
 (segment (start 183.92 80.24) (end 191.52 72.64) (width 0.5) (layer "B.Cu") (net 33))
 (segment (start 193.544 72.64) (end 193.548 72.644) (width 0.5) (layer "B.Cu") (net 33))
 (segment (start 182.85 80.24) (end 183.92 80.24) (width 0.5) (layer "B.Cu") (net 33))
 (segment (start 193.544 52.32) (end 186.44 52.32) (width 0.5) (layer "B.Cu") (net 25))
 (segment (start 184.428 57.38) (end 182.85 57.38) (width 0.5) (layer "B.Cu") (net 25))
 (segment (start 185.42 53.34) (end 185.42 56.388) (width 0.5) (layer "B.Cu") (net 25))
 (segment (start 186.44 52.32) (end 185.42 53.34) (width 0.5) (layer "B.Cu") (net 25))
 (segment (start 193.548 52.324) (end 193.544 52.32) (width 0.5) (layer "B.Cu") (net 25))
 (segment (start 185.42 56.388) (end 184.428 57.38) (width 0.5) (layer "B.Cu") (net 25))
 (segment (start 193.524 47.22) (end 193.548 47.244) (width 0.5) (layer "B.Cu") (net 21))
 (segment (start 182.85 47.22) (end 193.524 47.22) (width 0.5) (layer "B.Cu") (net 21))
 (segment (start 189.484 60.452) (end 189.992 59.944) (width 0.5) (layer "B.Cu") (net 28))
 (segment (start 182.85 67.54) (end 183.92 67.54) (width 0.5) (layer "B.Cu") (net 28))
 (segment (start 183.92 67.54) (end 189.484 61.976) (width 0.5) (layer "B.Cu") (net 28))
 (segment (start 189.992 59.944) (end 193.548 59.944) (width 0.5) (layer "B.Cu") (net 28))
 (segment (start 189.484 61.976) (end 189.484 60.452) (width 0.5) (layer "B.Cu") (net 28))
 (segment (start 193.544 67.56) (end 193.548 67.564) (width 0.5) (layer "B.Cu") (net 31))
 (segment (start 182.85 75.16) (end 183.92 75.16) (width 0.5) (layer "B.Cu") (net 31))
 (segment (start 183.92 75.16) (end 191.52 67.56) (width 0.5) (layer "B.Cu") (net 31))
 (segment (start 191.52 67.56) (end 193.544 67.56) (width 0.5) (layer "B.Cu") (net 31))
 (segment (start 193.548 54.864) (end 193.544 54.86) (width 0.5) (layer "B.Cu") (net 26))
 (segment (start 185.928 60.96) (end 184.428 62.46) (width 0.5) (layer "B.Cu") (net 26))
 (segment (start 193.544 54.86) (end 188.98 54.86) (width 0.5) (layer "B.Cu") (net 26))
 (segment (start 185.928 57.912) (end 185.928 60.96) (width 0.5) (layer "B.Cu") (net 26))
 (segment (start 184.428 62.46) (end 182.85 62.46) (width 0.5) (layer "B.Cu") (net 26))
 (segment (start 188.98 54.86) (end 185.928 57.912) (width 0.5) (layer "B.Cu") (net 26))
 (segment (start 151.15 62.25) (end 153.9 65) (width 0.5) (layer "B.Cu") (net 2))
 (segment (start 149.95 62.25) (end 151.15 62.25) (width 0.5) (layer "B.Cu") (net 2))
 (segment (start 153.9 65) (end 157.45 65) (width 0.5) (layer "B.Cu") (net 2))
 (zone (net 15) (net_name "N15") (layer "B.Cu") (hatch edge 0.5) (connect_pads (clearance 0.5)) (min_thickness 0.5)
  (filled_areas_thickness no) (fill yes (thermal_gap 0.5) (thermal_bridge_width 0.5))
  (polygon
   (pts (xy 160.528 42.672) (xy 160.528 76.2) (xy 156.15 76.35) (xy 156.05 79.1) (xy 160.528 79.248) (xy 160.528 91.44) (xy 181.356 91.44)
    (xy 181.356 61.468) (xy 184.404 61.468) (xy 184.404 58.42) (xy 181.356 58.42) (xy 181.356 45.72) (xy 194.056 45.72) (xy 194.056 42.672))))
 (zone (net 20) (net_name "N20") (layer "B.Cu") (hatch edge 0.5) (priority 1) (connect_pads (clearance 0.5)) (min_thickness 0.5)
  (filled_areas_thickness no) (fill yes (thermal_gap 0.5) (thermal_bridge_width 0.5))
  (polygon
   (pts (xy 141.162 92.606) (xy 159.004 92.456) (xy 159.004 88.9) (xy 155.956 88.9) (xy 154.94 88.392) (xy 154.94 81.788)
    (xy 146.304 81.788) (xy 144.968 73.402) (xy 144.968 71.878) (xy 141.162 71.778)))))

